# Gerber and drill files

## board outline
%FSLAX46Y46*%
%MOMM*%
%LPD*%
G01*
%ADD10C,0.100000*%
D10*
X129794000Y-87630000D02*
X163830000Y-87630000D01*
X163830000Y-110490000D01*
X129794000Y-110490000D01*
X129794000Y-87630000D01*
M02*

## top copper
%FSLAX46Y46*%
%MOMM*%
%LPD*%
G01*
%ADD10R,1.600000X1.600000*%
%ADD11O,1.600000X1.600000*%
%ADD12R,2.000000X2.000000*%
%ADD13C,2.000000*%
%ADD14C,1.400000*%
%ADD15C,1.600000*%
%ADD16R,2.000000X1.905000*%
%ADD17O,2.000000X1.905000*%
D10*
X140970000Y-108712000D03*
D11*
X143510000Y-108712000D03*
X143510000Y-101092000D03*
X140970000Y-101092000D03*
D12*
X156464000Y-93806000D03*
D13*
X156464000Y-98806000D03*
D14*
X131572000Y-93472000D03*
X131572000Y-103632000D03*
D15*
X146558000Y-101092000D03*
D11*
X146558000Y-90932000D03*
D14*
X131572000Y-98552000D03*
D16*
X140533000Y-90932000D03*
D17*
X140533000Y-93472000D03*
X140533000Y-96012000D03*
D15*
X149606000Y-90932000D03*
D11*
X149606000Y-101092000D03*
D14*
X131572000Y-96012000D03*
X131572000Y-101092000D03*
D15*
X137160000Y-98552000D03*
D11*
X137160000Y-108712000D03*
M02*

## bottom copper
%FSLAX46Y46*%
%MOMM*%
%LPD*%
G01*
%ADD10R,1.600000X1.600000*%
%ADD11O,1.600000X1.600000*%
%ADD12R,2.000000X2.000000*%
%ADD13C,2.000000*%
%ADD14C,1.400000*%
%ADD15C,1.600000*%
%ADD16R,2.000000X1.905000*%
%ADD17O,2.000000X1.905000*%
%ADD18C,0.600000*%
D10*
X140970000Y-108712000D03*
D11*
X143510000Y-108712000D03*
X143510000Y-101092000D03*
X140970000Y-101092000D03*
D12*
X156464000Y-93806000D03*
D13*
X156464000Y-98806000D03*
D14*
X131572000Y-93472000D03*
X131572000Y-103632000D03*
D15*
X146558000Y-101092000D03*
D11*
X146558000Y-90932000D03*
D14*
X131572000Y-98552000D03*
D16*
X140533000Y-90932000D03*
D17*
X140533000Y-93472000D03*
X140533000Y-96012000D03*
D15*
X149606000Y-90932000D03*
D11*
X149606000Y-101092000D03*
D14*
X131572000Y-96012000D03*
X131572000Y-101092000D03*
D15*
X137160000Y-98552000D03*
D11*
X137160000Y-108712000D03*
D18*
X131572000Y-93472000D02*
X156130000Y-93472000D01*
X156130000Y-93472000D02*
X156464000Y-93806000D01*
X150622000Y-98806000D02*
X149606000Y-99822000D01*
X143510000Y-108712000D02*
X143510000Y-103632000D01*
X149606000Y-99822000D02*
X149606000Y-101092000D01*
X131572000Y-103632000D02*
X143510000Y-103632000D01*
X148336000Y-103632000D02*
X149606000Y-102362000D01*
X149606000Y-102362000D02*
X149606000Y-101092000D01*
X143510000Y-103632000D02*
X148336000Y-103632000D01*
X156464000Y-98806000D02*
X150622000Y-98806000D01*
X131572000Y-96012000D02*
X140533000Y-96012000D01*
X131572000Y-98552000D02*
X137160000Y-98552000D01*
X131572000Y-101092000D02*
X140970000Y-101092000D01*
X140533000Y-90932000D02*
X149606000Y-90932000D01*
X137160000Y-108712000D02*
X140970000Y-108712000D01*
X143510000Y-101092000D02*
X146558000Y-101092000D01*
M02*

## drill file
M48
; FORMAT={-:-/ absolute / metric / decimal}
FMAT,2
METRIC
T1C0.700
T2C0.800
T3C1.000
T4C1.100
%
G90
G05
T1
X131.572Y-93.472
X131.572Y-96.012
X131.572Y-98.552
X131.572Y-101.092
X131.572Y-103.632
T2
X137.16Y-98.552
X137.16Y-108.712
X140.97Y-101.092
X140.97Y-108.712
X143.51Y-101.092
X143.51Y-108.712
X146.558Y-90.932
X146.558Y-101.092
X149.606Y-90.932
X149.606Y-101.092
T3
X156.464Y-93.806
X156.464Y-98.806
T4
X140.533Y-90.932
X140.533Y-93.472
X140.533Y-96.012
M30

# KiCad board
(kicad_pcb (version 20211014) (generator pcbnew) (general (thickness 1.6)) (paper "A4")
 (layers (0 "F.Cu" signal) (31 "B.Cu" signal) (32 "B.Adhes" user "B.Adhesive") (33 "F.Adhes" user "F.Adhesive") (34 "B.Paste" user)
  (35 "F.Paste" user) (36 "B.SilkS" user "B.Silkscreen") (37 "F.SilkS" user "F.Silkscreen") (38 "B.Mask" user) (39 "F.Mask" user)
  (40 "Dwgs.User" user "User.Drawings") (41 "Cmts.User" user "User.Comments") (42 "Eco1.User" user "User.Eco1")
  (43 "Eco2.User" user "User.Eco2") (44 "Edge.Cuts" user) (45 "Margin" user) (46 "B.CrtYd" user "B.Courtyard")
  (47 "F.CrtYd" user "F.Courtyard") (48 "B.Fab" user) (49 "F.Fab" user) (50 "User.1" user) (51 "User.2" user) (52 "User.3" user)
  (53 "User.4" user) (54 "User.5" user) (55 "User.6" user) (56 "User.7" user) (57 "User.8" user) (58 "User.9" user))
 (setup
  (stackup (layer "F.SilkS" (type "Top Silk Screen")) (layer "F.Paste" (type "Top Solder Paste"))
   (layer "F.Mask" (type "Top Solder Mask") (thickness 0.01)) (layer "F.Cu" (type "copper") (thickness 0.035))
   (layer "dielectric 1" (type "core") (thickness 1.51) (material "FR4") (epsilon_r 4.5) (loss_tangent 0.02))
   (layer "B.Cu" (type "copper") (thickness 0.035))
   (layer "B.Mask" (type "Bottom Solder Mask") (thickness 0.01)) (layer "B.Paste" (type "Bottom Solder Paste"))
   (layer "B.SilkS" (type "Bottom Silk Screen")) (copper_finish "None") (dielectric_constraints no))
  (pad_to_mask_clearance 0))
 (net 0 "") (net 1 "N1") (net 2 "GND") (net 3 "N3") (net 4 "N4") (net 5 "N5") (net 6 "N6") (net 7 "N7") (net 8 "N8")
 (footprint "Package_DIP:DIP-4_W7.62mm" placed (layer "F.Cu") (at 140.97 108.712 90)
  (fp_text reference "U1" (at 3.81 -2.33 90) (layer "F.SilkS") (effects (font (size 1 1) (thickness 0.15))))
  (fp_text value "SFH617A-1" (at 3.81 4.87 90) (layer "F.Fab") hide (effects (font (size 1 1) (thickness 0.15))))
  (pad "1" thru_hole rect locked (at 0 0 90) (size 1.6 1.6) (drill 0.8) (layers *.Cu *.Mask) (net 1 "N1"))
  (pad "2" thru_hole oval locked (at 0 2.54 90) (size 1.6 1.6) (drill 0.8) (layers *.Cu *.Mask) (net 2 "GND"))
  (pad "3" thru_hole oval locked (at 7.62 2.54 90) (size 1.6 1.6) (drill 0.8) (layers *.Cu *.Mask) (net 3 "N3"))
  (pad "4" thru_hole oval locked (at 7.62 0 90) (size 1.6 1.6) (drill 0.8) (layers *.Cu *.Mask) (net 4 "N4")))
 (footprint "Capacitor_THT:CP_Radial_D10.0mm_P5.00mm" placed (layer "F.Cu") (at 156.464 93.806 -90)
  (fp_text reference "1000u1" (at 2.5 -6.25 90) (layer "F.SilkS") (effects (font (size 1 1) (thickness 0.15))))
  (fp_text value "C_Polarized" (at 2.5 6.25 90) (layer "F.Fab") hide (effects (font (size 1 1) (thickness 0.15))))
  (pad "1" thru_hole rect locked (at 0 0 270) (size 2 2) (drill 1) (layers *.Cu *.Mask) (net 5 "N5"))
  (pad "2" thru_hole circle locked (at 5 0 270) (size 2 2) (drill 1) (layers *.Cu *.Mask) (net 2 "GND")))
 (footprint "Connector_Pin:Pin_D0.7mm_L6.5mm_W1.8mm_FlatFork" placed (layer "F.Cu") (at 131.572 93.472)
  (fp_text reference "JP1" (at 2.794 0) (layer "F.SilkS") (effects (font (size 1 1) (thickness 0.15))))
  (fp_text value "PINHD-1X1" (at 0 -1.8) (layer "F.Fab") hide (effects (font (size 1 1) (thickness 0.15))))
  (pad "1" thru_hole circle locked (at 0 0) (size 1.4 1.4) (drill 0.7) (layers *.Cu *.Mask) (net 5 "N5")))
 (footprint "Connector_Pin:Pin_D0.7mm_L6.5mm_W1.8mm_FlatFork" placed (layer "F.Cu") (at 131.572 103.632)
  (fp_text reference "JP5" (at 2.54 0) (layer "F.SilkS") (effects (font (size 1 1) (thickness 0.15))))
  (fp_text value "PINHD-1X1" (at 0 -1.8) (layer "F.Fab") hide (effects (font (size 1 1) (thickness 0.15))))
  (pad "1" thru_hole circle locked (at 0 0) (size 1.4 1.4) (drill 0.7) (layers *.Cu *.Mask) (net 2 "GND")))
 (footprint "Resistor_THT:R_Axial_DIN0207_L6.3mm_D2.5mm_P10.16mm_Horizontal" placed (layer "F.Cu") (at 146.558 101.092 90)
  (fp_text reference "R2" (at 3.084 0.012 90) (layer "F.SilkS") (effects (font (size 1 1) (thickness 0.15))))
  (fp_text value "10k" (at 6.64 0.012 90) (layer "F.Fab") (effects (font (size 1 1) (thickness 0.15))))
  (pad "1" thru_hole circle locked (at 0 0 90) (size 1.6 1.6) (drill 0.8) (layers *.Cu *.Mask) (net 3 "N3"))
  (pad "2" thru_hole oval locked (at 10.16 0 90) (size 1.6 1.6) (drill 0.8) (layers *.Cu *.Mask) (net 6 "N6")))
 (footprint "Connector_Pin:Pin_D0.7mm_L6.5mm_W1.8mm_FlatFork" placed (layer "F.Cu") (at 131.572 98.552)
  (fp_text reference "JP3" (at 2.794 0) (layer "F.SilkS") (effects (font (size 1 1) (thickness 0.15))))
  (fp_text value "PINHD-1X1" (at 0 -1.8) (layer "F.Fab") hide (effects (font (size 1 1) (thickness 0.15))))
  (pad "1" thru_hole circle locked (at 0 0) (size 1.4 1.4) (drill 0.7) (layers *.Cu *.Mask) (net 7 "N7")))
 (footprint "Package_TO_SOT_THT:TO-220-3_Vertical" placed (layer "F.Cu") (at 140.533 90.932 -90)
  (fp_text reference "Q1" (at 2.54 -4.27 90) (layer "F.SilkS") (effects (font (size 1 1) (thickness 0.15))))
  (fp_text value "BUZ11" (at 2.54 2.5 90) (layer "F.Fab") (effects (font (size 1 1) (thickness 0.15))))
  (pad "1" thru_hole rect locked (at 0 0 270) (size 1.905 2) (drill 1.1) (layers *.Cu *.Mask) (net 6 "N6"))
  (pad "2" thru_hole oval locked (at 2.54 0 270) (size 1.905 2) (drill 1.1) (layers *.Cu *.Mask) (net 5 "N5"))
  (pad "3" thru_hole oval locked (at 5.08 0 270) (size 1.905 2) (drill 1.1) (layers *.Cu *.Mask) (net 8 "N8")))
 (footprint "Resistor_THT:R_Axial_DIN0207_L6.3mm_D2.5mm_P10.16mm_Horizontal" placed (layer "F.Cu") (at 149.606 90.932 -90)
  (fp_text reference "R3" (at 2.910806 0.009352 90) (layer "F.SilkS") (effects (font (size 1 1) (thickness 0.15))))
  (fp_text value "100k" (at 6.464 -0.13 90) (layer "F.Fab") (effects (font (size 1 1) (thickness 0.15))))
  (pad "1" thru_hole circle locked (at 0 0 270) (size 1.6 1.6) (drill 0.8) (layers *.Cu *.Mask) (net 6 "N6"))
  (pad "2" thru_hole oval locked (at 10.16 0 270) (size 1.6 1.6) (drill 0.8) (layers *.Cu *.Mask) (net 2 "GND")))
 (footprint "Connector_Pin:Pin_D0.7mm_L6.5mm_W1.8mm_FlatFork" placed (layer "F.Cu") (at 131.572 96.012)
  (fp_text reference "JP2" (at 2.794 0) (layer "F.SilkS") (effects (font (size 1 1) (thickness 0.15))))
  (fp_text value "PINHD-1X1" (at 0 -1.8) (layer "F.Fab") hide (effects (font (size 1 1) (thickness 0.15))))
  (pad "1" thru_hole circle locked (at 0 0) (size 1.4 1.4) (drill 0.7) (layers *.Cu *.Mask) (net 8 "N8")))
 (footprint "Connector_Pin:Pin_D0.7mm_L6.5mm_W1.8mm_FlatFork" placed (layer "F.Cu") (at 131.572 101.092)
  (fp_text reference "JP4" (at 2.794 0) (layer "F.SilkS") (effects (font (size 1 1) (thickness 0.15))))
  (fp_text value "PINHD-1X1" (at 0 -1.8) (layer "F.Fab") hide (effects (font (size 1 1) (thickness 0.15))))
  (pad "1" thru_hole circle locked (at 0 0) (size 1.4 1.4) (drill 0.7) (layers *.Cu *.Mask) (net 4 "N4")))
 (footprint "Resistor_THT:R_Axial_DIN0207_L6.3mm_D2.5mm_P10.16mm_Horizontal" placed (layer "F.Cu") (at 137.16 98.552 -90)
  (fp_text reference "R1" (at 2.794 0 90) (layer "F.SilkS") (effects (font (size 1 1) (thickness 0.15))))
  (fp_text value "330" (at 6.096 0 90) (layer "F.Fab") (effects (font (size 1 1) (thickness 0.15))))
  (pad "1" thru_hole circle locked (at 0 0 270) (size 1.6 1.6) (drill 0.8) (layers *.Cu *.Mask) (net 7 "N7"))
  (pad "2" thru_hole oval locked (at 10.16 0 270) (size 1.6 1.6) (drill 0.8) (layers *.Cu *.Mask) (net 1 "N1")))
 (gr_rect (start 129.794 87.63) (end 163.83 110.49) (layer "Edge.Cuts") (width 0.1) (fill none))
 (segment (start 131.572 93.472) (end 156.13 93.472) (width 0.6) (layer "B.Cu") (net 5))
 (segment (start 156.13 93.472) (end 156.464 93.806) (width 0.6) (layer "B.Cu") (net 5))
 (segment (start 150.622 98.806) (end 149.606 99.822) (width 0.6) (layer "B.Cu") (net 2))
 (segment (start 143.51 108.712) (end 143.51 103.632) (width 0.6) (layer "B.Cu") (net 2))
 (segment (start 149.606 99.822) (end 149.606 101.092) (width 0.6) (layer "B.Cu") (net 2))
 (segment (start 131.572 103.632) (end 143.51 103.632) (width 0.6) (layer "B.Cu") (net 2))
 (segment (start 148.336 103.632) (end 149.606 102.362) (width 0.6) (layer "B.Cu") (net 2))
 (segment (start 149.606 102.362) (end 149.606 101.092) (width 0.6) (layer "B.Cu") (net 2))
 (segment (start 143.51 103.632) (end 148.336 103.632) (width 0.6) (layer "B.Cu") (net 2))
 (segment (start 156.464 98.806) (end 150.622 98.806) (width 0.6) (layer "B.Cu") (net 2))
 (segment (start 131.572 96.012) (end 140.533 96.012) (width 0.6) (layer "B.Cu") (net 8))
 (segment (start 131.572 98.552) (end 137.16 98.552) (width 0.6) (layer "B.Cu") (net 7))
 (segment (start 131.572 101.092) (end 140.97 101.092) (width 0.6) (layer "B.Cu") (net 4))
 (segment (start 140.533 90.932) (end 149.606 90.932) (width 0.6) (layer "B.Cu") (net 6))
 (segment (start 137.16 108.712) (end 140.97 108.712) (width 0.6) (layer "B.Cu") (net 1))
 (segment (start 143.51 101.092) (end 146.558 101.092) (width 0.6) (layer "B.Cu") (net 3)))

